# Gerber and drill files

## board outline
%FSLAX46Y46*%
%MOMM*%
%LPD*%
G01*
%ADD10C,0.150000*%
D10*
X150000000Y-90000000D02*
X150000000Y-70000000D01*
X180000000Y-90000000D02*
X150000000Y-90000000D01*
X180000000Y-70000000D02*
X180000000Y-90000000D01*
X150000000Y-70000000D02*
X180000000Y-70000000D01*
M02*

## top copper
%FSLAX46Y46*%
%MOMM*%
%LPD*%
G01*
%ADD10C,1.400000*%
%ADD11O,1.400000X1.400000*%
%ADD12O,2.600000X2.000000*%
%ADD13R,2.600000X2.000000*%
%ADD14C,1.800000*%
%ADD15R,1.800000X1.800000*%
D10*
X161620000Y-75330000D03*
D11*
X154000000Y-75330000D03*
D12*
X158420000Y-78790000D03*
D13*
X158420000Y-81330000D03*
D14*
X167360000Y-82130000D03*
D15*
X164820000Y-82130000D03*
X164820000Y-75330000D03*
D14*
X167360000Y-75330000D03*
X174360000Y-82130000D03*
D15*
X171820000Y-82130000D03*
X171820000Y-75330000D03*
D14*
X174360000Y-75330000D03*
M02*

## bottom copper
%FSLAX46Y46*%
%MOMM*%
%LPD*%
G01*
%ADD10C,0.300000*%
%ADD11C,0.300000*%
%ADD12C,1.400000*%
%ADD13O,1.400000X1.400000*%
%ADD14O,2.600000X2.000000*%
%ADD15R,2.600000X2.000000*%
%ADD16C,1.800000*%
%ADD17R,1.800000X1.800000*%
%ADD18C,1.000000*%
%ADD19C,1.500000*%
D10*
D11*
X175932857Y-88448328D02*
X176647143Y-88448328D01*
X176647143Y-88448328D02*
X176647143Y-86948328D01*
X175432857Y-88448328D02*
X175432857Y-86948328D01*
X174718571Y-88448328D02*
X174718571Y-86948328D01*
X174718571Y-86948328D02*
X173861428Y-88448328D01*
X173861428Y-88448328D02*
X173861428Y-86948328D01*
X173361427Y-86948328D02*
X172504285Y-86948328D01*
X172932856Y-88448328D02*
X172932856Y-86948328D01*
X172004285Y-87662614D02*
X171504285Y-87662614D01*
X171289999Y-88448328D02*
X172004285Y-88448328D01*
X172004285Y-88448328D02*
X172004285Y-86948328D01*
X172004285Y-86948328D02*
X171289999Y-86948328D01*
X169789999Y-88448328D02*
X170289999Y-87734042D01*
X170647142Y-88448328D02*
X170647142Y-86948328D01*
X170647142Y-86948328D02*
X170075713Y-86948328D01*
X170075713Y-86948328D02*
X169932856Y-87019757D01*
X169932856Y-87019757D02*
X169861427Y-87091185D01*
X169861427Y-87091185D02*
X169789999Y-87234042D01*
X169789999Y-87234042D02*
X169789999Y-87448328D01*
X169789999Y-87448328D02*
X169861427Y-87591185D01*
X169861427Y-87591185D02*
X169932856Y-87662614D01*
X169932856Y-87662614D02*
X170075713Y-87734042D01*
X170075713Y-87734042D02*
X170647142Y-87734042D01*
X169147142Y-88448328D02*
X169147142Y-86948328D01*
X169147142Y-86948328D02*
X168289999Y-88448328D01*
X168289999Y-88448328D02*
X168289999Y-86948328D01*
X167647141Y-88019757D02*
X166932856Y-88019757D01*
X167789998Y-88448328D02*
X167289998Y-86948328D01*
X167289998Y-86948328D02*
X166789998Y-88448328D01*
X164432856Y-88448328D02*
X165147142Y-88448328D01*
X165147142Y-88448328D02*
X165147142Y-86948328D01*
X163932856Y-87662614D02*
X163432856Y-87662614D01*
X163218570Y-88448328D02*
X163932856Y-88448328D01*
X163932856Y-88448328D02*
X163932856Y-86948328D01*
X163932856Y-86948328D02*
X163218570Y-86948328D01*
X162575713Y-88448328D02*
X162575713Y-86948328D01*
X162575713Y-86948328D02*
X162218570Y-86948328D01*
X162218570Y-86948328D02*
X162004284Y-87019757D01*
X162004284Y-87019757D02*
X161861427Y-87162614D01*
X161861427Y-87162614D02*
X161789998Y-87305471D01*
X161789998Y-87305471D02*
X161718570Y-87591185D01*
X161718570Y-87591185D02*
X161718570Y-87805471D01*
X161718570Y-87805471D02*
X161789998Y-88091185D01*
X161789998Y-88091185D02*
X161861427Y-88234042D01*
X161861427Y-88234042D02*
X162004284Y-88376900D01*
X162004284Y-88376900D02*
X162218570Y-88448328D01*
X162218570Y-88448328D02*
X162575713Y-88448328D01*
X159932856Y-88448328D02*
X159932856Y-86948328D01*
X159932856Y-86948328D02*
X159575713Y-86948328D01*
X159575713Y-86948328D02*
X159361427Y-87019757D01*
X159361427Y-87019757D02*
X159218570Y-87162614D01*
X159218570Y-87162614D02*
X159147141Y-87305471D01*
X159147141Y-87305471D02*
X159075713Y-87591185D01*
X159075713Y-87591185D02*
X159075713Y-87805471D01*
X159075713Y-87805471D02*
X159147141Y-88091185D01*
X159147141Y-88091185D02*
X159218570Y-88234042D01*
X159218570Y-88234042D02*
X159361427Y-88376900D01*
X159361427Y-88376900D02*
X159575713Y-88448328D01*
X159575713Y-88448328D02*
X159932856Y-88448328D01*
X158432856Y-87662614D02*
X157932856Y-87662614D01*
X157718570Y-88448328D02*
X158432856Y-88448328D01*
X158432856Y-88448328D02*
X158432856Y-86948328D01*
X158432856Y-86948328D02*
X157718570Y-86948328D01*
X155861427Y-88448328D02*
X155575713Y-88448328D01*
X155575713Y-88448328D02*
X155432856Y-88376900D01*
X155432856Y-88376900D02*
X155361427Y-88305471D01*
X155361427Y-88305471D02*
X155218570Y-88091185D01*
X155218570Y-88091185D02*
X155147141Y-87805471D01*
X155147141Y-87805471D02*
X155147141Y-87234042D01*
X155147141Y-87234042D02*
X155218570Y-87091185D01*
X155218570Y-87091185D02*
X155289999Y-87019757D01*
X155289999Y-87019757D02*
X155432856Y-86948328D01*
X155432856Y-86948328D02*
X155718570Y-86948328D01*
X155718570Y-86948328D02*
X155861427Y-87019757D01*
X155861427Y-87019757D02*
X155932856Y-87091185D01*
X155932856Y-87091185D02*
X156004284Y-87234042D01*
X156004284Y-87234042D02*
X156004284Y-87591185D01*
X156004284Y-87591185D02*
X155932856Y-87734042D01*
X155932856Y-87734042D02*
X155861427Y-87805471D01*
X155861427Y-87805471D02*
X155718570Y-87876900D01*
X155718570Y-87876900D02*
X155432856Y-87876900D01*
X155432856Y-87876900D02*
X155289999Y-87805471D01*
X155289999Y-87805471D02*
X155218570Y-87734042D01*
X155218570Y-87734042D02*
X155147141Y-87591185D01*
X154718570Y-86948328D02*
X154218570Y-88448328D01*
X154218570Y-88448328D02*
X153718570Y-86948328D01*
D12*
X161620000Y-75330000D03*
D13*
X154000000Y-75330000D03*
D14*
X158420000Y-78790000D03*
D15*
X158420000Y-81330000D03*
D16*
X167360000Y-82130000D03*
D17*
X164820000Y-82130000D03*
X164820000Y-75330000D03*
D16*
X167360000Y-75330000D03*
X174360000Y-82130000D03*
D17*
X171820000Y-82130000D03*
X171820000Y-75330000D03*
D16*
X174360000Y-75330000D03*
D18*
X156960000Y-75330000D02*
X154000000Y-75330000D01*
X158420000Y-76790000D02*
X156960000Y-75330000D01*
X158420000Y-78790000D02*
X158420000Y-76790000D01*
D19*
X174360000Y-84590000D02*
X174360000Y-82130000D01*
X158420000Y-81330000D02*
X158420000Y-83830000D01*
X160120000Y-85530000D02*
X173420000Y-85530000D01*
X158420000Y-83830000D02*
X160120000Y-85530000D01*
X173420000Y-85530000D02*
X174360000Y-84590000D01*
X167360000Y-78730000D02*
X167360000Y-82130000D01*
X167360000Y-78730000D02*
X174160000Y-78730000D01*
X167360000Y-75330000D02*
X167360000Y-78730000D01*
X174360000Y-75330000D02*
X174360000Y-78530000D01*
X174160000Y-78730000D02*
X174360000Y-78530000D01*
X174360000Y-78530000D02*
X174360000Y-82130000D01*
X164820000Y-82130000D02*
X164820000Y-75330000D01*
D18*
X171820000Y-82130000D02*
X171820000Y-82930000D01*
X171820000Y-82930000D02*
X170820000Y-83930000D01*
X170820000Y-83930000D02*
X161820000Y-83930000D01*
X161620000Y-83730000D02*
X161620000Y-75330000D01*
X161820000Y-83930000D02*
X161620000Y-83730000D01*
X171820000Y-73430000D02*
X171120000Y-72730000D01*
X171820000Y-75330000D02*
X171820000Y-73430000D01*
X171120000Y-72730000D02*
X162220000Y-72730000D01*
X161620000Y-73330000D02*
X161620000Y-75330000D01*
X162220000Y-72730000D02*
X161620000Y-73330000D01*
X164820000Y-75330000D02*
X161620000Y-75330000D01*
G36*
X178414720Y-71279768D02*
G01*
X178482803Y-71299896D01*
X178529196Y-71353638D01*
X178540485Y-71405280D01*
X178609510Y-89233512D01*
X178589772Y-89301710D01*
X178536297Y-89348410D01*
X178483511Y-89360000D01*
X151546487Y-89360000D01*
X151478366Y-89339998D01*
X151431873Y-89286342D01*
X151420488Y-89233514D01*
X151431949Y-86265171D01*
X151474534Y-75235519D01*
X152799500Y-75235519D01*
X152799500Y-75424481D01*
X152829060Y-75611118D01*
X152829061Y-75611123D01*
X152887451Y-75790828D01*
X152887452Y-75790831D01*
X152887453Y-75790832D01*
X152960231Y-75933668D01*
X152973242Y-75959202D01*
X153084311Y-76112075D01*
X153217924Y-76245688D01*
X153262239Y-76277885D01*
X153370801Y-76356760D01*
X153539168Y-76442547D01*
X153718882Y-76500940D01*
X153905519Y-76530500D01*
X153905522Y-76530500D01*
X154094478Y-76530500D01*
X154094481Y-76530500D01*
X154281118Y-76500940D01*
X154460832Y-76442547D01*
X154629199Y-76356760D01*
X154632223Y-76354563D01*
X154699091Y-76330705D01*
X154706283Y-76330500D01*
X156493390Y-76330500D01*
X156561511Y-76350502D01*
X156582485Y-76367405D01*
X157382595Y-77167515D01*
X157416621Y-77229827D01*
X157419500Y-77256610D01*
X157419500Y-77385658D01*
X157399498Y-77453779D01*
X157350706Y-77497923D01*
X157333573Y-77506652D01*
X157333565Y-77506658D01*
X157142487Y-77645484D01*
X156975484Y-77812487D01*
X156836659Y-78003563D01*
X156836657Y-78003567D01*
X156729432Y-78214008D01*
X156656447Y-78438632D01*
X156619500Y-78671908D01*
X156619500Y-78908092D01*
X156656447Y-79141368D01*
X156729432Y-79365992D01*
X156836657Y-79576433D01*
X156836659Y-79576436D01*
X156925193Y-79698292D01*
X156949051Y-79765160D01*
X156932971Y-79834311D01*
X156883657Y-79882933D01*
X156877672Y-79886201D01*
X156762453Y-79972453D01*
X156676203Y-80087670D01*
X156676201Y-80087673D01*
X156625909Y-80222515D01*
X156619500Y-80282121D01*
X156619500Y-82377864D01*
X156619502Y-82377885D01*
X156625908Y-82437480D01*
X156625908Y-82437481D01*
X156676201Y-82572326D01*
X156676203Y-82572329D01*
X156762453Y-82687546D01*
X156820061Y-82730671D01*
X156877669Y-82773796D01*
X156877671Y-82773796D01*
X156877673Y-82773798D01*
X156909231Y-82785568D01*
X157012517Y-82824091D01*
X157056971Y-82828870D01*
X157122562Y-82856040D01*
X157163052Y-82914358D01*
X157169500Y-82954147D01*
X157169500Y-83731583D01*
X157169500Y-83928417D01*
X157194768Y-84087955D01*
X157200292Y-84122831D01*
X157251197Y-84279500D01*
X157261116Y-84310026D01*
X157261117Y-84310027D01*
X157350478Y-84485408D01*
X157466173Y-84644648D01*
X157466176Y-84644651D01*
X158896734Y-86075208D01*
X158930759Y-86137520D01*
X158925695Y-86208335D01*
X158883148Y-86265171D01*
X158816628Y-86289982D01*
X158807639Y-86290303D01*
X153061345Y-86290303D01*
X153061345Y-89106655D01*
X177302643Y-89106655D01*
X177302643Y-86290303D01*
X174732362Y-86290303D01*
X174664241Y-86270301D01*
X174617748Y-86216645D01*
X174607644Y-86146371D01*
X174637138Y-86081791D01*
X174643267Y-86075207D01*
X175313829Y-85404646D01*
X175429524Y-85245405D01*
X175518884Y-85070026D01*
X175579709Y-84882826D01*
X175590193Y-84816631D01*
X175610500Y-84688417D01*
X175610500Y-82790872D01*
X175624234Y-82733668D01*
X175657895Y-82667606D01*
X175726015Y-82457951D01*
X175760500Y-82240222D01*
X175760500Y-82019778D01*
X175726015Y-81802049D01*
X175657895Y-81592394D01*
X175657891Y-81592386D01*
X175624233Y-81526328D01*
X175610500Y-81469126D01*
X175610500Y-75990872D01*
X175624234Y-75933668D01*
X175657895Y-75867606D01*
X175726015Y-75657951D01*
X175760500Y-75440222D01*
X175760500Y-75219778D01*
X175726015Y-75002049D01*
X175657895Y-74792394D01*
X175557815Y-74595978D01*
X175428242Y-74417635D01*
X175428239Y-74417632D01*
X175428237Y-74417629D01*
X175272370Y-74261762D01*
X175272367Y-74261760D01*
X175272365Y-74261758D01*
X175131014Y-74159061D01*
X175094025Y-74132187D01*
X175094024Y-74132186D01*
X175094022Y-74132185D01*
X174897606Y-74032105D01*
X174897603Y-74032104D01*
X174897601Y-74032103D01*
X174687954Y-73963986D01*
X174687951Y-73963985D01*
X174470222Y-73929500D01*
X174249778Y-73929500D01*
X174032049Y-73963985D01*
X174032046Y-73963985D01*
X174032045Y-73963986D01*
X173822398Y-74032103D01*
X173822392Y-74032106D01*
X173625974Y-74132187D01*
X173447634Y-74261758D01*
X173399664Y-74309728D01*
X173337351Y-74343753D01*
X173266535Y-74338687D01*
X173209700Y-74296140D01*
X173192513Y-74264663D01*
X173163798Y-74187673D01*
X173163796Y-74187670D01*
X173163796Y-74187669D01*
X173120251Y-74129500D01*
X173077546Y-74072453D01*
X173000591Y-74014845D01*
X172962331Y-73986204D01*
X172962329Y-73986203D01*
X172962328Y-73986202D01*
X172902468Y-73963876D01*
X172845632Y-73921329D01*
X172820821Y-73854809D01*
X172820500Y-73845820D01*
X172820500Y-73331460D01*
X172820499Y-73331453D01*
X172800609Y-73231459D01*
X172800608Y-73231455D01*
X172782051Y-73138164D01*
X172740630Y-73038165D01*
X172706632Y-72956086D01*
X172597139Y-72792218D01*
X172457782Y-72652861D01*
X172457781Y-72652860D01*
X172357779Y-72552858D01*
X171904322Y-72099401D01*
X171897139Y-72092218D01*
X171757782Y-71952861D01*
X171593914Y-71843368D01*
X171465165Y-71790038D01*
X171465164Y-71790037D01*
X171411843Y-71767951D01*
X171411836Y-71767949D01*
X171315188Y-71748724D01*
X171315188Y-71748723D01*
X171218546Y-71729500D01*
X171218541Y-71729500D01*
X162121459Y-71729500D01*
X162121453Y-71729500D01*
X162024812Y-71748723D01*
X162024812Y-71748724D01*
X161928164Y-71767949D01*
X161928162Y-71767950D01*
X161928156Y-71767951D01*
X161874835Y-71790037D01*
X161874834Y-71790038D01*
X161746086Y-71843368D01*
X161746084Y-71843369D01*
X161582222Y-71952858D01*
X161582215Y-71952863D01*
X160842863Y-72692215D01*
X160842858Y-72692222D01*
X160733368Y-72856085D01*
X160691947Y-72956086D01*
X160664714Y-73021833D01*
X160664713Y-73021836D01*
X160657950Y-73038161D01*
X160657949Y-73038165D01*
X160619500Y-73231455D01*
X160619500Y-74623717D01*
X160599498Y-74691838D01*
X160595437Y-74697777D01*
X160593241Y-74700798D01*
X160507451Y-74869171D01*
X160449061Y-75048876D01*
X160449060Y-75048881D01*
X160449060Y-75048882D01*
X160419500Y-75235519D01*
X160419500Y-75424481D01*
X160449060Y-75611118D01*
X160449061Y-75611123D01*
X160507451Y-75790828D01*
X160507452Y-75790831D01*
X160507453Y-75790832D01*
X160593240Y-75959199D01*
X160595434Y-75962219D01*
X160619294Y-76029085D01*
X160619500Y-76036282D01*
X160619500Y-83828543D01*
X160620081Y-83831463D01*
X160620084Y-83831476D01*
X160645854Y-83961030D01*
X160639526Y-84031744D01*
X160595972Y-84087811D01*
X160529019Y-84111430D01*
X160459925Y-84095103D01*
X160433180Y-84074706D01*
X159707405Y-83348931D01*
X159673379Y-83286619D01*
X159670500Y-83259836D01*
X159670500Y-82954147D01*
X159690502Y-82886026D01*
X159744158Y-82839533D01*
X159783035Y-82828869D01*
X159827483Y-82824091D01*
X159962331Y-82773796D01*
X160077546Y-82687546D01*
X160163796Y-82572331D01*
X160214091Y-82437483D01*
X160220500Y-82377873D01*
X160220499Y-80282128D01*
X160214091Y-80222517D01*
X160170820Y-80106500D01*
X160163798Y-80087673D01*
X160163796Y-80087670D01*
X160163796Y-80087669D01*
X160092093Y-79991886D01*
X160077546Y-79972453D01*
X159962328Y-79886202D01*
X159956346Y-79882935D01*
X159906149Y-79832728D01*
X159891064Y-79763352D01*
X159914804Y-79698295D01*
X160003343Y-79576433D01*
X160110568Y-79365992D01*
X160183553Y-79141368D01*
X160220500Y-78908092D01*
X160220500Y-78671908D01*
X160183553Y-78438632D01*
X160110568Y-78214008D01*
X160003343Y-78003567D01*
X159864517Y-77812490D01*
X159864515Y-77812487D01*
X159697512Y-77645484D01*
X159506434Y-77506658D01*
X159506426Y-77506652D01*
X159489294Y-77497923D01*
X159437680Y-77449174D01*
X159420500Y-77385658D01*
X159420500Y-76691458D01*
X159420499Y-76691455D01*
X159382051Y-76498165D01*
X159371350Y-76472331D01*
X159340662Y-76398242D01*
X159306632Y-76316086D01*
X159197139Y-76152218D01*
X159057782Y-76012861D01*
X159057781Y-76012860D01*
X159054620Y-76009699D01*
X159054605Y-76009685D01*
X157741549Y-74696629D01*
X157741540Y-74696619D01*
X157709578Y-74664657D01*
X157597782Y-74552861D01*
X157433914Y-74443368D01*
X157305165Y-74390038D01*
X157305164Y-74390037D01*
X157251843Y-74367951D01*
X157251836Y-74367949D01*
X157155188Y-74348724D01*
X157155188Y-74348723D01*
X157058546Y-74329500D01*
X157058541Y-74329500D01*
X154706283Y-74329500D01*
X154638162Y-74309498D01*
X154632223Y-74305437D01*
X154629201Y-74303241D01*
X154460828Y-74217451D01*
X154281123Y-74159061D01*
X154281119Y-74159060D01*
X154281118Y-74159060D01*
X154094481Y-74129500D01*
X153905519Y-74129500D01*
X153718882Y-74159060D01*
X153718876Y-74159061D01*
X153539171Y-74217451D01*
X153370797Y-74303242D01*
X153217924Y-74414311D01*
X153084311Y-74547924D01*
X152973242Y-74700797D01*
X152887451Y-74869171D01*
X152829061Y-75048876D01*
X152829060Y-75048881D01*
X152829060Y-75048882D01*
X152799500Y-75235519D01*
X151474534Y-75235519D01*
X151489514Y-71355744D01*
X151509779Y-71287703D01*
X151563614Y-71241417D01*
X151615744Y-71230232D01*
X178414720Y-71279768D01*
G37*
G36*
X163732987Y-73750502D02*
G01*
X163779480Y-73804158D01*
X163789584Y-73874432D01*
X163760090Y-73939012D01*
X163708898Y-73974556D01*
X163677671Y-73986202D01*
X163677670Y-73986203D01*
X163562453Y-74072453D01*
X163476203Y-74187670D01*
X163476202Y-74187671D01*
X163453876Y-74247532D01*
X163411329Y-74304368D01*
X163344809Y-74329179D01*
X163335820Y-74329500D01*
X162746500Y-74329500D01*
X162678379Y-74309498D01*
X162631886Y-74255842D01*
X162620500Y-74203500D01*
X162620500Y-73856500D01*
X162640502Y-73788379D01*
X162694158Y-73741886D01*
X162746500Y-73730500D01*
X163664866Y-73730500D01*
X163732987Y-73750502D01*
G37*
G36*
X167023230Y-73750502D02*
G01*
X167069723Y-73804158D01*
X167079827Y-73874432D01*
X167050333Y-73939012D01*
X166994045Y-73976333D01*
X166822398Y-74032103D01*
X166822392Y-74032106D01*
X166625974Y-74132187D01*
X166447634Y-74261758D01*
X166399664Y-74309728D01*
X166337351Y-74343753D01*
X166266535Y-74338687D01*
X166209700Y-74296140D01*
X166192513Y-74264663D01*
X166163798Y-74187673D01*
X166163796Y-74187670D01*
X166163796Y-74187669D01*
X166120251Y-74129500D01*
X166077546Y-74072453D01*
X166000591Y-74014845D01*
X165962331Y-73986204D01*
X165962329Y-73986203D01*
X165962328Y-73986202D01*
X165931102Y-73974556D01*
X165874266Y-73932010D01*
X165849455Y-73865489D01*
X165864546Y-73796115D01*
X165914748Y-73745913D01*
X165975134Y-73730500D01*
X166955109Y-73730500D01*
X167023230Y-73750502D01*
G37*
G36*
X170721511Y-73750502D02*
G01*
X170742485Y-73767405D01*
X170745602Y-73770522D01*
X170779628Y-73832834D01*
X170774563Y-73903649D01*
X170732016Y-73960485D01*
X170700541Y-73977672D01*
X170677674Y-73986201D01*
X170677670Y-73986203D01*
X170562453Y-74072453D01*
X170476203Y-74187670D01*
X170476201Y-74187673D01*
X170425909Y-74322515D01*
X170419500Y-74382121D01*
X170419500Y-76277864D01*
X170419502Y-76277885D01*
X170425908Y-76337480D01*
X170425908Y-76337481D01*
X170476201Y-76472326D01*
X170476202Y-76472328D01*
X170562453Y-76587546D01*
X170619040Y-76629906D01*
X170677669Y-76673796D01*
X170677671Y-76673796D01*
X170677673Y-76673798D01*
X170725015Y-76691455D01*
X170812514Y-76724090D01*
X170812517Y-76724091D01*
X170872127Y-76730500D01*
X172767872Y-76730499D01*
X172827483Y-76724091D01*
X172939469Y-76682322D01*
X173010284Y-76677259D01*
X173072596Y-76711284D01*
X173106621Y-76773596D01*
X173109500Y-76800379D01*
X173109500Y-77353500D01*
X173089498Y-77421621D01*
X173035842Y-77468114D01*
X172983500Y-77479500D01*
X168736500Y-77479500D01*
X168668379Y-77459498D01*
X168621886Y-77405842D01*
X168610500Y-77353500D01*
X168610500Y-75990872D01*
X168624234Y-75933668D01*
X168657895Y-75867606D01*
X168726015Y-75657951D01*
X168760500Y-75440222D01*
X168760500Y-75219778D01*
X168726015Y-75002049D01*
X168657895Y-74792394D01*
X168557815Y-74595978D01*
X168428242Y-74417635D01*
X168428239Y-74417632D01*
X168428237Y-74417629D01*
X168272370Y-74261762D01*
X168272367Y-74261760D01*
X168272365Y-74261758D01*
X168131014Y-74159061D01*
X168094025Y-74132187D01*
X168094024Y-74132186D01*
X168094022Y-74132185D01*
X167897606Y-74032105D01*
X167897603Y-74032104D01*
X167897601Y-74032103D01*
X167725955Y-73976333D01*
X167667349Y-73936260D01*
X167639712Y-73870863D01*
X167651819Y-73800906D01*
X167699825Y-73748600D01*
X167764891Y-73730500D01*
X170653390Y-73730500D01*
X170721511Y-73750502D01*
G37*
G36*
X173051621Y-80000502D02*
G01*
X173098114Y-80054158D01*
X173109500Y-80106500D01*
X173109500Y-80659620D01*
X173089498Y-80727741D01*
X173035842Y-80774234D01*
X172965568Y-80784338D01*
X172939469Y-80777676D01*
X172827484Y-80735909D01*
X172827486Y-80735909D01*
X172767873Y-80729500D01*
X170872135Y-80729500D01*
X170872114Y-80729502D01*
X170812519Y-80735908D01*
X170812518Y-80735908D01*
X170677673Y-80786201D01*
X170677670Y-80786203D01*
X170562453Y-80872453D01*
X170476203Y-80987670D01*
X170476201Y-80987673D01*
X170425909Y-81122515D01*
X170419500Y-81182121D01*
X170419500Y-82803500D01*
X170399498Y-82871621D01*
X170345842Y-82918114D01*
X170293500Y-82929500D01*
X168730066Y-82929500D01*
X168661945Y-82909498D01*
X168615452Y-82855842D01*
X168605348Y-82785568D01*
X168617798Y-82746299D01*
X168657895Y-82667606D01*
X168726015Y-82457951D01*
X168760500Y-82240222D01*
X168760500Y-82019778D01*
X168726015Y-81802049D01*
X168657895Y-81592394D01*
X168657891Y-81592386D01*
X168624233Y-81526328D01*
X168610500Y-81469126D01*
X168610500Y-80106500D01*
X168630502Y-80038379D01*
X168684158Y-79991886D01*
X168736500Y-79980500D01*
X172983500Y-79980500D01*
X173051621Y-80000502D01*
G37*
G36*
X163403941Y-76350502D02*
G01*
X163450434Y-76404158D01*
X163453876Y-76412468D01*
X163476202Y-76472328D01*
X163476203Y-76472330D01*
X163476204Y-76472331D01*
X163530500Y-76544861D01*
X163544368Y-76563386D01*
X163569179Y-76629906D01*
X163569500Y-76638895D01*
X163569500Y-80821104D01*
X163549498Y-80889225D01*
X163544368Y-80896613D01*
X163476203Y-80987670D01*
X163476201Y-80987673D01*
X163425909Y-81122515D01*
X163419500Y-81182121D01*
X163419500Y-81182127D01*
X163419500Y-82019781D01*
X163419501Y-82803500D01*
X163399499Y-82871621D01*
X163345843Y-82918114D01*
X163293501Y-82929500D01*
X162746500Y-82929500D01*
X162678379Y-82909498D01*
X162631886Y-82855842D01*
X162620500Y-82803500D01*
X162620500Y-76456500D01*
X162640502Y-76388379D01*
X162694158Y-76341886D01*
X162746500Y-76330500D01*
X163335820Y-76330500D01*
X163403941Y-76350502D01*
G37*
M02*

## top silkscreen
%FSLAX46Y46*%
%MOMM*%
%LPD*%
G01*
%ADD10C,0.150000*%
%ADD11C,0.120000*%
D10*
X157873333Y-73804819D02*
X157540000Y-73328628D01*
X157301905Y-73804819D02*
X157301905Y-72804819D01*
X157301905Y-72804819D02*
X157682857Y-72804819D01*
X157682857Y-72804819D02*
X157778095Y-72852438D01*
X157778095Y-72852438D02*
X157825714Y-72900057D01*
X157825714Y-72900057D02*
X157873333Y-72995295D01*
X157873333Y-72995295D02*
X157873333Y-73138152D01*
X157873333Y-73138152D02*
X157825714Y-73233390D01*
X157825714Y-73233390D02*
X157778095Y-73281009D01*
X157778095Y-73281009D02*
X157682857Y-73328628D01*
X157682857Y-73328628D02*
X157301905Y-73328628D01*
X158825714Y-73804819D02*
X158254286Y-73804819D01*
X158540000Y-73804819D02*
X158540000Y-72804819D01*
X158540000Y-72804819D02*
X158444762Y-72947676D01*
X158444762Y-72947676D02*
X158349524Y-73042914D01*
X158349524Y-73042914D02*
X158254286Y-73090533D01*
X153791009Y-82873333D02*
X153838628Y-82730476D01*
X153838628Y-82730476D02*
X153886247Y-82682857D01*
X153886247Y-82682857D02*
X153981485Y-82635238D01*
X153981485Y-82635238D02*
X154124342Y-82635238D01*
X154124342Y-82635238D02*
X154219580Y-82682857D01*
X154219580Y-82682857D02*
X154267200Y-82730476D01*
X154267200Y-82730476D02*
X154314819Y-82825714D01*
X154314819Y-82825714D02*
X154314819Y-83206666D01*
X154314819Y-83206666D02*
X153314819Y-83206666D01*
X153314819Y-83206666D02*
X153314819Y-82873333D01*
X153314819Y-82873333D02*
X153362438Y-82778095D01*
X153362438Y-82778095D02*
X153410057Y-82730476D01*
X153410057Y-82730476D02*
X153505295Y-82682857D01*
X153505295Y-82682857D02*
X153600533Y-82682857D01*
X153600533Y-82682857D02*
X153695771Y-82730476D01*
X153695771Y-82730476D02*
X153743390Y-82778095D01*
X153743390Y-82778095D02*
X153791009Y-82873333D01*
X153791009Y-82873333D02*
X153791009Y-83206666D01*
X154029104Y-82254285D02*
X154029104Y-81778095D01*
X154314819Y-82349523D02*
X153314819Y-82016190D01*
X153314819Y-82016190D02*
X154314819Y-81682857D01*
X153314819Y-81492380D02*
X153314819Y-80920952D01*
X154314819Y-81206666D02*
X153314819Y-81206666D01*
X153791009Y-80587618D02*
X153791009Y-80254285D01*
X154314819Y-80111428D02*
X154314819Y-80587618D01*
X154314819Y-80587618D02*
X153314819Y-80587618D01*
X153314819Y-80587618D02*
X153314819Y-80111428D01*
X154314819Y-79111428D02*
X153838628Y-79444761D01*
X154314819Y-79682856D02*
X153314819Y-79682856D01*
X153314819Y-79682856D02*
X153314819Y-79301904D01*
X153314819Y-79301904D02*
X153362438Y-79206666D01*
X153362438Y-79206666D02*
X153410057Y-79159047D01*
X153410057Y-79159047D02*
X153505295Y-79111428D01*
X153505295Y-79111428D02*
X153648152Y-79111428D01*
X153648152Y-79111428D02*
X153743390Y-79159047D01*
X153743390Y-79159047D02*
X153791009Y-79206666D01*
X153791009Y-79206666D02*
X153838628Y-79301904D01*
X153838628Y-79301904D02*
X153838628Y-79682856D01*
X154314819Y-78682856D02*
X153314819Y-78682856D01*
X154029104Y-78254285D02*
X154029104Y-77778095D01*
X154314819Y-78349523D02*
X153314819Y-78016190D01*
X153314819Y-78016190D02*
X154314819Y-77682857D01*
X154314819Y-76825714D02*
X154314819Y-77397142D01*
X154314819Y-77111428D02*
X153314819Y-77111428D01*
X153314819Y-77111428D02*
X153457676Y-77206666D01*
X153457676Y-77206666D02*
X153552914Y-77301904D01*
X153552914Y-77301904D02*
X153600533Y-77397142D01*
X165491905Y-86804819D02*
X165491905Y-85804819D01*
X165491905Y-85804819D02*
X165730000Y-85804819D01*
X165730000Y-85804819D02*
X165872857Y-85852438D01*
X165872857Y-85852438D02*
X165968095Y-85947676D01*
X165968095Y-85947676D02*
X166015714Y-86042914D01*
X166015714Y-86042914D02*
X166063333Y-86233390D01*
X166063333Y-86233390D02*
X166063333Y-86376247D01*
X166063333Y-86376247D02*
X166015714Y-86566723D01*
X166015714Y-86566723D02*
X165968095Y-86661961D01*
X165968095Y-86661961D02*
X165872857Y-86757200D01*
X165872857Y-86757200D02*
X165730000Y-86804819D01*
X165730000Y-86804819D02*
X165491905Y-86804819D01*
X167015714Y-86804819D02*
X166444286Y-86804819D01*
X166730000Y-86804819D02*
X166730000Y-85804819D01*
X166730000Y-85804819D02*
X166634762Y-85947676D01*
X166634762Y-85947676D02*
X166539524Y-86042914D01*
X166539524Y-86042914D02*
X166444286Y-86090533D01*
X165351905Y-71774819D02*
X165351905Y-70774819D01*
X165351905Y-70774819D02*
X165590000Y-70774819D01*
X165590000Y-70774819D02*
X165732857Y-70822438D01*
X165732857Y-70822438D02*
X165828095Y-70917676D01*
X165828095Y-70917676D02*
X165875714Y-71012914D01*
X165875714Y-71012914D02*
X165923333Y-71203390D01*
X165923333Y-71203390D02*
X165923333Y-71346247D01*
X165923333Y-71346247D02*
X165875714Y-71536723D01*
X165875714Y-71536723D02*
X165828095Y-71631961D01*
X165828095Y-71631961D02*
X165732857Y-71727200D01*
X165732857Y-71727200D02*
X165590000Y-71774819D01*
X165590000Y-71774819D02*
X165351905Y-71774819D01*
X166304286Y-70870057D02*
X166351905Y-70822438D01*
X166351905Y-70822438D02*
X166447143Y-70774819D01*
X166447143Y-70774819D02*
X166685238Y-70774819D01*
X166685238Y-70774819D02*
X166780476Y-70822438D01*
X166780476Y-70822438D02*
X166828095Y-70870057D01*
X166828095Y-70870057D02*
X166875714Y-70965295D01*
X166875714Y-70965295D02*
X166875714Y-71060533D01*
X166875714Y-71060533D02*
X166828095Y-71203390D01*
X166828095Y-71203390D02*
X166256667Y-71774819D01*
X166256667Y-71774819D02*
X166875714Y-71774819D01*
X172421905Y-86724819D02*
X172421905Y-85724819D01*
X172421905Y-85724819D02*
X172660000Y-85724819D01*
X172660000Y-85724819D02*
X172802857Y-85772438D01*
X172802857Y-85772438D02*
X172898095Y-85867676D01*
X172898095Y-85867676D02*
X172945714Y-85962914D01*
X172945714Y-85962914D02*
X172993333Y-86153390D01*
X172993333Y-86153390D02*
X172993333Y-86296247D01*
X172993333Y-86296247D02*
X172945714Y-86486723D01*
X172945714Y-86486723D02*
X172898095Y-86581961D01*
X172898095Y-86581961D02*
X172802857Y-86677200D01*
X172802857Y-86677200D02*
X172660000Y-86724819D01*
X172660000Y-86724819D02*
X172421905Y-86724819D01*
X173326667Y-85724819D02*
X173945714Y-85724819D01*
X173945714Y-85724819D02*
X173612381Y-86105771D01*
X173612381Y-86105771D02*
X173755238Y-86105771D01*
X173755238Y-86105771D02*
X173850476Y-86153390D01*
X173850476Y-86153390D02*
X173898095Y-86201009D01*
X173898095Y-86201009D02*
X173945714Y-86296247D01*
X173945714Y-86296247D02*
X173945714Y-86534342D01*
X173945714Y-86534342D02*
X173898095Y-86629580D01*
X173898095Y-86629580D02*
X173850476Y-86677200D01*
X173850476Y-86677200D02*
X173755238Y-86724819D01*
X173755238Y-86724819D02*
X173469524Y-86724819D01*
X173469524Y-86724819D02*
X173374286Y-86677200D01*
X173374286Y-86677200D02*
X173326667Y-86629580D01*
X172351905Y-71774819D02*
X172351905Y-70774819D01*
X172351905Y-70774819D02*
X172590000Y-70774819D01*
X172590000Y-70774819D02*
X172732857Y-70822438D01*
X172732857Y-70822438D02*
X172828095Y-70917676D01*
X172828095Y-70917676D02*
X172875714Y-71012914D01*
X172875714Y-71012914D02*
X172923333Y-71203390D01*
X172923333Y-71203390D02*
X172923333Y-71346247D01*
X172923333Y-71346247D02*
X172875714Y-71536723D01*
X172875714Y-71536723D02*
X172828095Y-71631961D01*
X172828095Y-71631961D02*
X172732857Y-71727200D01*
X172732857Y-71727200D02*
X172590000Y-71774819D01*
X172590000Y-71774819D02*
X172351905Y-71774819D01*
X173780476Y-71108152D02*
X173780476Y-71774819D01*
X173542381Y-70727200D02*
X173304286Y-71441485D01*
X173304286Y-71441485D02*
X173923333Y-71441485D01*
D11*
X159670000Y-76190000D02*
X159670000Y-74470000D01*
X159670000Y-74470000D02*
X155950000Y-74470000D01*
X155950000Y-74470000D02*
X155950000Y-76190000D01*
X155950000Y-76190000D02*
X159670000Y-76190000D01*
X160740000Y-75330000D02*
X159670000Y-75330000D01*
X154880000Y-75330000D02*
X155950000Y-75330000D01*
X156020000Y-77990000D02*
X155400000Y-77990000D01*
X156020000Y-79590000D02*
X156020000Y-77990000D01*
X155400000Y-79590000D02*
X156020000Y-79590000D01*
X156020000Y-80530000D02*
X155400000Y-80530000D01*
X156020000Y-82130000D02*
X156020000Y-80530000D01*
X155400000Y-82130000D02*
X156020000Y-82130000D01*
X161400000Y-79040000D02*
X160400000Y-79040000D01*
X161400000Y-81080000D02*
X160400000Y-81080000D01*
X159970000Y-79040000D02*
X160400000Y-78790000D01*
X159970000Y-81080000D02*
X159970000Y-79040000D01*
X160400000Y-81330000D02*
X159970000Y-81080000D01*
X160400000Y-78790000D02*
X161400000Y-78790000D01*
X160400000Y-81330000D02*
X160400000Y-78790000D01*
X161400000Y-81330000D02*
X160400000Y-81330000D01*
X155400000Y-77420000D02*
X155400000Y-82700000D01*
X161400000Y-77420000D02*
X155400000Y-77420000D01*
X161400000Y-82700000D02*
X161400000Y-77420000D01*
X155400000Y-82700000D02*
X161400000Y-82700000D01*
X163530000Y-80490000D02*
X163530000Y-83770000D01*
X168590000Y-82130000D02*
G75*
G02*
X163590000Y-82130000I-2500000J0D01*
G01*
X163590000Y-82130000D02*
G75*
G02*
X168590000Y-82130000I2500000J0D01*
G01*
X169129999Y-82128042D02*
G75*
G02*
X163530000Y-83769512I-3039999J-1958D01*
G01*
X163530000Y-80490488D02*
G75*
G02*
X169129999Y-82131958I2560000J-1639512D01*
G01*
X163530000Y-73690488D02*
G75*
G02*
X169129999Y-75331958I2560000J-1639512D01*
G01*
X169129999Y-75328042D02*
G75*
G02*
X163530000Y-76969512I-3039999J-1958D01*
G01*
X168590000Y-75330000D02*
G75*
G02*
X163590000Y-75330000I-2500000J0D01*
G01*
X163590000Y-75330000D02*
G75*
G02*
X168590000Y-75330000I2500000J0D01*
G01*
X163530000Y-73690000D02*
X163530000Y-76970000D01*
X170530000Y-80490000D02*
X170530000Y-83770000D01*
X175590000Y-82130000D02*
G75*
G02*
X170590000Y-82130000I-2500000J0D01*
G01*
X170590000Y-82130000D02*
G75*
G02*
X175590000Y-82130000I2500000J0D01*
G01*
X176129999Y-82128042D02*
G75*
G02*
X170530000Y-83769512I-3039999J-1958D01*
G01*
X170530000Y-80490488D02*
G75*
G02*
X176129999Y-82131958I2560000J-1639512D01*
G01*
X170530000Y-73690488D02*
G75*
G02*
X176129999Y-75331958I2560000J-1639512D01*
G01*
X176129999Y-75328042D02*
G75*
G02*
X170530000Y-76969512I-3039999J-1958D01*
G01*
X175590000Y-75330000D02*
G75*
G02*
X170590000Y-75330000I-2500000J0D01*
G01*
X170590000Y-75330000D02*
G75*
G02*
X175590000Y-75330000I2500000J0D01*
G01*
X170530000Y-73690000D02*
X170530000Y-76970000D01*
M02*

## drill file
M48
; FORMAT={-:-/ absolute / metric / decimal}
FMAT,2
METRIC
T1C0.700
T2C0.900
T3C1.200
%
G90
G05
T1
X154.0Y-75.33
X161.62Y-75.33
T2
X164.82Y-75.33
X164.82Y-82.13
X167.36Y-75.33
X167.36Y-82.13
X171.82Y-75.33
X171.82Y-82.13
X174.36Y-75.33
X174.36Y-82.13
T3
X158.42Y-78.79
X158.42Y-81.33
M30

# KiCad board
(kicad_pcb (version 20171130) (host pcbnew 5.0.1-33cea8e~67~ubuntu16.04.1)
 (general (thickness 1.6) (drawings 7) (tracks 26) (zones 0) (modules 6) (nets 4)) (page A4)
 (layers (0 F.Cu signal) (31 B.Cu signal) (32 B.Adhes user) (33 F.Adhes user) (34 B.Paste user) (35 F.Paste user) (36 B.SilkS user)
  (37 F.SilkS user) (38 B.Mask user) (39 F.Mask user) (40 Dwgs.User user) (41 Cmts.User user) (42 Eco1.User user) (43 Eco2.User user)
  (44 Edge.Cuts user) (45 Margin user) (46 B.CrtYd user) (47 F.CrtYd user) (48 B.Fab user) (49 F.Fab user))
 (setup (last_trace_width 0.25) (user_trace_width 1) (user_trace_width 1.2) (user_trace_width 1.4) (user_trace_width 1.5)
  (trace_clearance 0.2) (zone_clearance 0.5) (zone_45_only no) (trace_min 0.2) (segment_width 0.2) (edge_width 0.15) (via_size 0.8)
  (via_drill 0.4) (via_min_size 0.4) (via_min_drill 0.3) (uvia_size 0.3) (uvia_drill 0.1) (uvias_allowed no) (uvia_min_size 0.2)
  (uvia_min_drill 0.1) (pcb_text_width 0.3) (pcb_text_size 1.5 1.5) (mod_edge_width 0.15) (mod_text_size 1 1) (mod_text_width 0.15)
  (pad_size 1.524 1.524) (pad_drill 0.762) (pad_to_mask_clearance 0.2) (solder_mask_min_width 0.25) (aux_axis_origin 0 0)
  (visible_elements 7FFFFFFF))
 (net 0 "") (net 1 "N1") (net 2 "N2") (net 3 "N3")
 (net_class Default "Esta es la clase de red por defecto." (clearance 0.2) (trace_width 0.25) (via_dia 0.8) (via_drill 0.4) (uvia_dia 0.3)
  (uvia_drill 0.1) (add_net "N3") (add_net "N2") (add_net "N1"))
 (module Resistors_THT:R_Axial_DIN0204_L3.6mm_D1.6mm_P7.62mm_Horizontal (layer F.Cu) (at 161.62 75.33 180)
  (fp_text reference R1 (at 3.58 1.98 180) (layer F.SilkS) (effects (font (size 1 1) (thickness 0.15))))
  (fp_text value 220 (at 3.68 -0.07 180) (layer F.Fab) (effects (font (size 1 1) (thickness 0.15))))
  (fp_line (start 1.95 -0.86) (end 1.95 0.86) (layer F.SilkS) (width 0.12))
  (fp_line (start 1.95 0.86) (end 5.67 0.86) (layer F.SilkS) (width 0.12))
  (fp_line (start 5.67 0.86) (end 5.67 -0.86) (layer F.SilkS) (width 0.12))
  (fp_line (start 5.67 -0.86) (end 1.95 -0.86) (layer F.SilkS) (width 0.12))
  (fp_line (start 0.88 0) (end 1.95 0) (layer F.SilkS) (width 0.12))
  (fp_line (start 6.74 0) (end 5.67 0) (layer F.SilkS) (width 0.12))
  (pad 1 thru_hole circle (at 0 0 180) (size 1.4 1.4) (drill 0.7) (layers *.Cu *.Mask) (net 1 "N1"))
  (pad 2 thru_hole oval (at 7.62 0 180) (size 1.4 1.4) (drill 0.7) (layers *.Cu *.Mask) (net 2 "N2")))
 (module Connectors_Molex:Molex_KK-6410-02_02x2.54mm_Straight (layer F.Cu) (at 158.42 81.33 90)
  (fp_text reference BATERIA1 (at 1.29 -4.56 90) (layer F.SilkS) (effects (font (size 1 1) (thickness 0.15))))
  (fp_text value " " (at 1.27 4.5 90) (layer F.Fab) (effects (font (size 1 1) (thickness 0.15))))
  (fp_line (start 3.34 -2.4) (end 3.34 -3.02) (layer F.SilkS) (width 0.12))
  (fp_line (start 1.74 -2.4) (end 3.34 -2.4) (layer F.SilkS) (width 0.12))
  (fp_line (start 1.74 -3.02) (end 1.74 -2.4) (layer F.SilkS) (width 0.12))
  (fp_line (start 0.8 -2.4) (end 0.8 -3.02) (layer F.SilkS) (width 0.12))
  (fp_line (start -0.8 -2.4) (end 0.8 -2.4) (layer F.SilkS) (width 0.12))
  (fp_line (start -0.8 -3.02) (end -0.8 -2.4) (layer F.SilkS) (width 0.12))
  (fp_line (start 2.29 2.98) (end 2.29 1.98) (layer F.SilkS) (width 0.12))
  (fp_line (start 0.25 2.98) (end 0.25 1.98) (layer F.SilkS) (width 0.12))
  (fp_line (start 2.29 1.55) (end 2.54 1.98) (layer F.SilkS) (width 0.12))
  (fp_line (start 0.25 1.55) (end 2.29 1.55) (layer F.SilkS) (width 0.12))
  (fp_line (start 0 1.98) (end 0.25 1.55) (layer F.SilkS) (width 0.12))
  (fp_line (start 2.54 1.98) (end 2.54 2.98) (layer F.SilkS) (width 0.12))
  (fp_line (start 0 1.98) (end 2.54 1.98) (layer F.SilkS) (width 0.12))
  (fp_line (start 0 2.98) (end 0 1.98) (layer F.SilkS) (width 0.12))
  (fp_line (start 3.91 -3.02) (end -1.37 -3.02) (layer F.SilkS) (width 0.12))
  (fp_line (start 3.91 2.98) (end 3.91 -3.02) (layer F.SilkS) (width 0.12))
  (fp_line (start -1.37 2.98) (end 3.91 2.98) (layer F.SilkS) (width 0.12))
  (fp_line (start -1.37 -3.02) (end -1.37 2.98) (layer F.SilkS) (width 0.12))
  (pad 2 thru_hole oval (at 2.54 0 90) (size 2 2.6) (drill 1.2) (layers *.Cu *.Mask) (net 2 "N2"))
  (pad 1 thru_hole rect (at 0 0 90) (size 2 2.6) (drill 1.2) (layers *.Cu *.Mask) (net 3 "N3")))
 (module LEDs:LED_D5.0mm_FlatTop (layer F.Cu) (at 164.82 82.13)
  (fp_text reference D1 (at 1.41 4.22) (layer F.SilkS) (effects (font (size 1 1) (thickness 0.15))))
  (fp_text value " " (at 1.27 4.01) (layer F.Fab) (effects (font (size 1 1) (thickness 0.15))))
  (fp_line (start -1.29 -1.64) (end -1.29 1.64) (layer F.SilkS) (width 0.12))
  (fp_circle (center 1.27 0) (end 3.77 0) (layer F.SilkS) (width 0.12))
  (fp_arc (start 1.27 0) (end -1.29 1.639512) (angle -147.4) (layer F.SilkS) (width 0.12))
  (fp_arc (start 1.27 0) (end -1.29 -1.639512) (angle 147.4) (layer F.SilkS) (width 0.12))
  (pad 2 thru_hole circle (at 2.54 0) (size 1.8 1.8) (drill 0.9) (layers *.Cu *.Mask) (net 3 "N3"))
  (pad 1 thru_hole rect (at 0 0) (size 1.8 1.8) (drill 0.9) (layers *.Cu *.Mask) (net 1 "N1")))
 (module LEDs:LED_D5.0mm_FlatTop (layer F.Cu) (at 164.82 75.33)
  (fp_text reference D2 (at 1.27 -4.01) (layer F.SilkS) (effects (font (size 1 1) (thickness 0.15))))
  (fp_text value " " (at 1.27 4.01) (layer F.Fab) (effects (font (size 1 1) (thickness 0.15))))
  (fp_arc (start 1.27 0) (end -1.29 -1.639512) (angle 147.4) (layer F.SilkS) (width 0.12))
  (fp_arc (start 1.27 0) (end -1.29 1.639512) (angle -147.4) (layer F.SilkS) (width 0.12))
  (fp_circle (center 1.27 0) (end 3.77 0) (layer F.SilkS) (width 0.12))
  (fp_line (start -1.29 -1.64) (end -1.29 1.64) (layer F.SilkS) (width 0.12))
  (pad 1 thru_hole rect (at 0 0) (size 1.8 1.8) (drill 0.9) (layers *.Cu *.Mask) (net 1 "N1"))
  (pad 2 thru_hole circle (at 2.54 0) (size 1.8 1.8) (drill 0.9) (layers *.Cu *.Mask) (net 3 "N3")))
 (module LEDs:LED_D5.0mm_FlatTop (layer F.Cu) (at 171.82 82.13)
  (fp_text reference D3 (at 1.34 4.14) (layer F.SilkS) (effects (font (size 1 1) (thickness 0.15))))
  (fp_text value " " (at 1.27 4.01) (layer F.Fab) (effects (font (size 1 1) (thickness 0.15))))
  (fp_line (start -1.29 -1.64) (end -1.29 1.64) (layer F.SilkS) (width 0.12))
  (fp_circle (center 1.27 0) (end 3.77 0) (layer F.SilkS) (width 0.12))
  (fp_arc (start 1.27 0) (end -1.29 1.639512) (angle -147.4) (layer F.SilkS) (width 0.12))
  (fp_arc (start 1.27 0) (end -1.29 -1.639512) (angle 147.4) (layer F.SilkS) (width 0.12))
  (pad 2 thru_hole circle (at 2.54 0) (size 1.8 1.8) (drill 0.9) (layers *.Cu *.Mask) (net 3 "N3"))
  (pad 1 thru_hole rect (at 0 0) (size 1.8 1.8) (drill 0.9) (layers *.Cu *.Mask) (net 1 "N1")))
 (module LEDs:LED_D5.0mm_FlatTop (layer F.Cu) (at 171.82 75.33)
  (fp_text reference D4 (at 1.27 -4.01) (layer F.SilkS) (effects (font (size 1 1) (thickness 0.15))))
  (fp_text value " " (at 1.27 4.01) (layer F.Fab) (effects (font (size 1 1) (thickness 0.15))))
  (fp_arc (start 1.27 0) (end -1.29 -1.639512) (angle 147.4) (layer F.SilkS) (width 0.12))
  (fp_arc (start 1.27 0) (end -1.29 1.639512) (angle -147.4) (layer F.SilkS) (width 0.12))
  (fp_circle (center 1.27 0) (end 3.77 0) (layer F.SilkS) (width 0.12))
  (fp_line (start -1.29 -1.64) (end -1.29 1.64) (layer F.SilkS) (width 0.12))
  (pad 1 thru_hole rect (at 0 0) (size 1.8 1.8) (drill 0.9) (layers *.Cu *.Mask) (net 1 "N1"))
  (pad 2 thru_hole circle (at 2.54 0) (size 1.8 1.8) (drill 0.9) (layers *.Cu *.Mask) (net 3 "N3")))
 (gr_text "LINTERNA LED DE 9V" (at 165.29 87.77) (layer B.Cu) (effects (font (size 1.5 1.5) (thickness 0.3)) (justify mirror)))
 (gr_line (start 150 90) (end 150 70) (layer Edge.Cuts) (width 0.15))
 (gr_line (start 180 90) (end 150 90) (layer Edge.Cuts) (width 0.15))
 (gr_line (start 180 70) (end 180 90) (layer Edge.Cuts) (width 0.15))
 (gr_line (start 150 70) (end 180 70) (layer Edge.Cuts) (width 0.15))
 (segment (start 156.96 75.33) (end 154 75.33) (width 1) (layer B.Cu) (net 2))
 (segment (start 158.42 76.79) (end 156.96 75.33) (width 1) (layer B.Cu) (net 2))
 (segment (start 158.42 78.79) (end 158.42 76.79) (width 1) (layer B.Cu) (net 2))
 (segment (start 174.36 84.59) (end 174.36 82.13) (width 1.5) (layer B.Cu) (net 3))
 (segment (start 158.42 81.33) (end 158.42 83.83) (width 1.5) (layer B.Cu) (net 3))
 (segment (start 160.12 85.53) (end 173.42 85.53) (width 1.5) (layer B.Cu) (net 3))
 (segment (start 158.42 83.83) (end 160.12 85.53) (width 1.5) (layer B.Cu) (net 3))
 (segment (start 173.42 85.53) (end 174.36 84.59) (width 1.5) (layer B.Cu) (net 3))
 (segment (start 167.36 78.73) (end 167.36 82.13) (width 1.5) (layer B.Cu) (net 3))
 (segment (start 167.36 78.73) (end 174.16 78.73) (width 1.5) (layer B.Cu) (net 3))
 (segment (start 167.36 75.33) (end 167.36 78.73) (width 1.5) (layer B.Cu) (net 3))
 (segment (start 174.36 75.33) (end 174.36 78.53) (width 1.5) (layer B.Cu) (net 3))
 (segment (start 174.16 78.73) (end 174.36 78.53) (width 1.5) (layer B.Cu) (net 3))
 (segment (start 174.36 78.53) (end 174.36 82.13) (width 1.5) (layer B.Cu) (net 3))
 (segment (start 164.82 82.13) (end 164.82 75.33) (width 1.5) (layer B.Cu) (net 1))
 (segment (start 171.82 82.13) (end 171.82 82.93) (width 1) (layer B.Cu) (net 1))
 (segment (start 171.82 82.93) (end 170.82 83.93) (width 1) (layer B.Cu) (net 1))
 (segment (start 170.82 83.93) (end 161.82 83.93) (width 1) (layer B.Cu) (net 1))
 (segment (start 161.62 83.73) (end 161.62 75.33) (width 1) (layer B.Cu) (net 1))
 (segment (start 161.82 83.93) (end 161.62 83.73) (width 1) (layer B.Cu) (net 1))
 (segment (start 171.82 73.43) (end 171.12 72.73) (width 1) (layer B.Cu) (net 1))
 (segment (start 171.82 75.33) (end 171.82 73.43) (width 1) (layer B.Cu) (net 1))
 (segment (start 171.12 72.73) (end 162.22 72.73) (width 1) (layer B.Cu) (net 1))
 (segment (start 161.62 73.33) (end 161.62 75.33) (width 1) (layer B.Cu) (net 1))
 (segment (start 162.22 72.73) (end 161.62 73.33) (width 1) (layer B.Cu) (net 1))
 (segment (start 164.82 75.33) (end 161.62 75.33) (width 1) (layer B.Cu) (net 1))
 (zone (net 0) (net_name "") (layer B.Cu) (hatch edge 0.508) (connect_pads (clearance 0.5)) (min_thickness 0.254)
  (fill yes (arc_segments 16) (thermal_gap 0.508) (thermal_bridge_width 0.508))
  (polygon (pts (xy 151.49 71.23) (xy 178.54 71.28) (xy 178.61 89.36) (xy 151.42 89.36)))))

